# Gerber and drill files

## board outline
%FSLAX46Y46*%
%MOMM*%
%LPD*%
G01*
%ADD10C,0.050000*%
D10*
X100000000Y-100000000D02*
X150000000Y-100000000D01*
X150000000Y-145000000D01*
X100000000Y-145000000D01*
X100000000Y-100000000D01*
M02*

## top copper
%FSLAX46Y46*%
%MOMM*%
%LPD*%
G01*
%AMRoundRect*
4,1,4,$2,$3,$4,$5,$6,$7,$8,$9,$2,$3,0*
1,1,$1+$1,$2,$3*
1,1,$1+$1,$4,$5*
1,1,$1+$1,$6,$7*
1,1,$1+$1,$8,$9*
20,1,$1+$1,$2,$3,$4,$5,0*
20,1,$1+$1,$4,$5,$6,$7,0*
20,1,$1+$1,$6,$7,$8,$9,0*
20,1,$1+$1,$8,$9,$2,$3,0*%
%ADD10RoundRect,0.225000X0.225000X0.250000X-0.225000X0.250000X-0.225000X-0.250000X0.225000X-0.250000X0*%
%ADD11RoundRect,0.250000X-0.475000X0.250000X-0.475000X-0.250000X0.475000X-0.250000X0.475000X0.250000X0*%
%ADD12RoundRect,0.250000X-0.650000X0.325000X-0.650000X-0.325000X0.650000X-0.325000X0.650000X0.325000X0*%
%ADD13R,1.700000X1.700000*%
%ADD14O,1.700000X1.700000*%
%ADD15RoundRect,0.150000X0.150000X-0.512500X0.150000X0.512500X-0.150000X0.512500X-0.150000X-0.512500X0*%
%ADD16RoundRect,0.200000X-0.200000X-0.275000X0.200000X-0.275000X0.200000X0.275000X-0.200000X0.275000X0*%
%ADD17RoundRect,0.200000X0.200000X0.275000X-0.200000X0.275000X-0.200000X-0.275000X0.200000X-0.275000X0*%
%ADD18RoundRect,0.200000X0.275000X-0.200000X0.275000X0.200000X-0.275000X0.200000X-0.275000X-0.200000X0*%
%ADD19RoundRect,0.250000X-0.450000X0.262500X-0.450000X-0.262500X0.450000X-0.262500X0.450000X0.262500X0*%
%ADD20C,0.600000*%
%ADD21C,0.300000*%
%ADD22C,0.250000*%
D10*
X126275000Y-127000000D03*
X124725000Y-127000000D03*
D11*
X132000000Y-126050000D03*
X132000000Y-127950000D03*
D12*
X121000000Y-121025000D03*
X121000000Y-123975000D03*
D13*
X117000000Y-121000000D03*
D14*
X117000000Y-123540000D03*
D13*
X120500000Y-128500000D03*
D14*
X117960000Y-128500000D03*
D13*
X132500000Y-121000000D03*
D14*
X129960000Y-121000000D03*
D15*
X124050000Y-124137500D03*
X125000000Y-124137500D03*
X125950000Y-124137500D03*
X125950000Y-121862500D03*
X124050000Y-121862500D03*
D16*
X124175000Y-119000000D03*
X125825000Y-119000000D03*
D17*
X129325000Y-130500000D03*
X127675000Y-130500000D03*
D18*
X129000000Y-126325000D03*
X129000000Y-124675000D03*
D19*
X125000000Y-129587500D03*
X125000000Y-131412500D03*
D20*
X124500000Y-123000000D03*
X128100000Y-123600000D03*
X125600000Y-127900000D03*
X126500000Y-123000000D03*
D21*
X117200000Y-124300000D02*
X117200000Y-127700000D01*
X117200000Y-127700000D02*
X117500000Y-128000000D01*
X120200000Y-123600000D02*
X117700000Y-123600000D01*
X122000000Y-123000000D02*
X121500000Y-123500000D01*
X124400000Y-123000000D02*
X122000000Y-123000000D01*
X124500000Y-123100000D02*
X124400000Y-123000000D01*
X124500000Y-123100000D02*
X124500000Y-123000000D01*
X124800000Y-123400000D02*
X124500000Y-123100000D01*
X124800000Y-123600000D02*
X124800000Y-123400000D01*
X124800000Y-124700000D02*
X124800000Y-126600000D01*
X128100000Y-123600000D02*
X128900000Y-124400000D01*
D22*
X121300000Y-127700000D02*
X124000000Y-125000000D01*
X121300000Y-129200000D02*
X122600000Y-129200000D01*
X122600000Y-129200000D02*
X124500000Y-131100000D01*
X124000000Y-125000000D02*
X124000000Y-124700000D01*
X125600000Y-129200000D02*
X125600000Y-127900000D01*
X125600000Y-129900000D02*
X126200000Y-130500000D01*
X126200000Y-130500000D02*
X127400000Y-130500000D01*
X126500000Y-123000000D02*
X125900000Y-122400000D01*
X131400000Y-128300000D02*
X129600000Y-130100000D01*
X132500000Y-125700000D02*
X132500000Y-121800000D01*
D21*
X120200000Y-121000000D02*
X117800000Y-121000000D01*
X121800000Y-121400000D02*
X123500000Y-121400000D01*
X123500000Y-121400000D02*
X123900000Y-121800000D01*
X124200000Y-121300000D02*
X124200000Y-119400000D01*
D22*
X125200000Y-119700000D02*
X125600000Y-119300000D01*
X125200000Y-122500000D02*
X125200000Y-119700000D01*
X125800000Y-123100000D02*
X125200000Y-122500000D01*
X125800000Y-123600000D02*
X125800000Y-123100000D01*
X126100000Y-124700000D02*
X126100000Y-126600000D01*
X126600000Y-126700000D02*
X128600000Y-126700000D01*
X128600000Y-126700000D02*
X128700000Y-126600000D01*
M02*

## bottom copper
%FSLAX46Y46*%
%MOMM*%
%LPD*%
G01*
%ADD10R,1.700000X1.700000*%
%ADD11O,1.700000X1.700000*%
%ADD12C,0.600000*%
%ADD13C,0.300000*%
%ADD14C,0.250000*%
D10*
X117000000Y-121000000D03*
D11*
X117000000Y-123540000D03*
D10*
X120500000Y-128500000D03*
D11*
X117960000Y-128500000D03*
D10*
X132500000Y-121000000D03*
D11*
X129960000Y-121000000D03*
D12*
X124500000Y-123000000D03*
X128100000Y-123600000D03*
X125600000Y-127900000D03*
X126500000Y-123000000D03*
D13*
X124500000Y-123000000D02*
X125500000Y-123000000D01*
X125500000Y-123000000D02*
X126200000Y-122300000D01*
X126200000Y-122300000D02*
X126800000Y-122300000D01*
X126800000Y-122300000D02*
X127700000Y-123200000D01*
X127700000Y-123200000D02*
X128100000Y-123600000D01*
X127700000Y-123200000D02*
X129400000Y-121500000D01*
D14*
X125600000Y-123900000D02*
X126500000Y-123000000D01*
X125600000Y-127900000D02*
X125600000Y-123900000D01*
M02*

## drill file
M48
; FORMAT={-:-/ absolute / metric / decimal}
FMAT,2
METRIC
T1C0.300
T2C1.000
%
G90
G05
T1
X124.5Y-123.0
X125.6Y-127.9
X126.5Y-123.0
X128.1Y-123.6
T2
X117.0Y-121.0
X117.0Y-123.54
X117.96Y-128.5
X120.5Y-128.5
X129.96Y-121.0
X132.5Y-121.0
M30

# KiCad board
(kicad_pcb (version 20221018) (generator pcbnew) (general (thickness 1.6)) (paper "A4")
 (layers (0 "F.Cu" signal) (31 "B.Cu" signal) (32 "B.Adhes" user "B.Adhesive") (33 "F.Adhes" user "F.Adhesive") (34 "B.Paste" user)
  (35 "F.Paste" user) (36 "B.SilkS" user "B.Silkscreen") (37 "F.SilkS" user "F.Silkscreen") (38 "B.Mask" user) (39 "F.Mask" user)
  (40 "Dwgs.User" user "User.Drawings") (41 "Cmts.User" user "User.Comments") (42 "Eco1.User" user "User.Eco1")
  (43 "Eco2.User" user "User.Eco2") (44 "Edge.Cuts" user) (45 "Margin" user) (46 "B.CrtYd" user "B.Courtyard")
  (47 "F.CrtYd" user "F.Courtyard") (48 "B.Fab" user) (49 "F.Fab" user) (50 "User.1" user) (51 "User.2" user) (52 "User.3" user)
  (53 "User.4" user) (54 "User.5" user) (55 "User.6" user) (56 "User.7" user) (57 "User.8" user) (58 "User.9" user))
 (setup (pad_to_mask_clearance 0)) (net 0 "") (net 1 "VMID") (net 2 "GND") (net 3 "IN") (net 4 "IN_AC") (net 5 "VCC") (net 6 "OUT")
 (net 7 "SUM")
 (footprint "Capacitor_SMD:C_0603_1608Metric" (layer "F.Cu") (at 125.5 127 180)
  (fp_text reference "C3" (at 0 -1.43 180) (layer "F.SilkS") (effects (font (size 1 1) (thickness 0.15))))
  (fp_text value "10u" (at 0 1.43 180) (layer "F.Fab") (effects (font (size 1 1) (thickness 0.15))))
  (pad "1" smd roundrect (at -0.775 0 180) (size 0.9 0.95) (layers "F.Cu" "F.Paste" "F.Mask") (roundrect_rratio 0.25) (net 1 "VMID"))
  (pad "2" smd roundrect (at 0.775 0 180) (size 0.9 0.95) (layers "F.Cu" "F.Paste" "F.Mask") (roundrect_rratio 0.25) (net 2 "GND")))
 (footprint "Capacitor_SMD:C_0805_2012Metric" (layer "F.Cu") (at 132 127 -90)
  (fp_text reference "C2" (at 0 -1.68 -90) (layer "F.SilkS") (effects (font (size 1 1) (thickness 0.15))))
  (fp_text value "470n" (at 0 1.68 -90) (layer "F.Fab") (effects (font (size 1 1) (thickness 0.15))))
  (pad "1" smd roundrect (at -0.95 0 270) (size 1 1.45) (layers "F.Cu" "F.Paste" "F.Mask") (roundrect_rratio 0.25) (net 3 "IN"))
  (pad "2" smd roundrect (at 0.95 0 270) (size 1 1.45) (layers "F.Cu" "F.Paste" "F.Mask") (roundrect_rratio 0.25) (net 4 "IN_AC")))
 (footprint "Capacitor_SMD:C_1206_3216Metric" (layer "F.Cu") (at 121 122.5 -90)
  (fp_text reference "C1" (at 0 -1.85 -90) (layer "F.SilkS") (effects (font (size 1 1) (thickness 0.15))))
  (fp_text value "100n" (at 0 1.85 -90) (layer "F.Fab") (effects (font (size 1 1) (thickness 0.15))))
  (pad "1" smd roundrect (at -1.475 0 270) (size 1.15 1.8) (layers "F.Cu" "F.Paste" "F.Mask") (roundrect_rratio 0.217391) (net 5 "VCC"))
  (pad "2" smd roundrect (at 1.475 0 270) (size 1.15 1.8) (layers "F.Cu" "F.Paste" "F.Mask") (roundrect_rratio 0.217391) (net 2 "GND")))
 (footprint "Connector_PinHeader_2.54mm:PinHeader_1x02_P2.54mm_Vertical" (layer "F.Cu") (at 117 121)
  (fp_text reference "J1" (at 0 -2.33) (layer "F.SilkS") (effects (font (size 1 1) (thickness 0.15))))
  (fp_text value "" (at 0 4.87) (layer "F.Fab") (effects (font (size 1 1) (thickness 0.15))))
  (pad "1" thru_hole rect (at 0 0) (size 1.7 1.7) (drill 1) (layers "*.Cu" "*.Mask") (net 5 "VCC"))
  (pad "2" thru_hole oval (at 0 2.54) (size 1.7 1.7) (drill 1) (layers "*.Cu" "*.Mask") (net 2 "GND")))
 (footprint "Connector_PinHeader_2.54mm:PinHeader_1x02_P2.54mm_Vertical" (layer "F.Cu") (at 120.5 128.5 -90)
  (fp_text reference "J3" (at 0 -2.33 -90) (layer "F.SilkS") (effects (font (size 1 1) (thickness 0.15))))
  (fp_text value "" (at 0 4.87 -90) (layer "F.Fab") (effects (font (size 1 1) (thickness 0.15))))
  (pad "1" thru_hole rect (at 0 0 270) (size 1.7 1.7) (drill 1) (layers "*.Cu" "*.Mask") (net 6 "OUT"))
  (pad "2" thru_hole oval (at 0 2.54 270) (size 1.7 1.7) (drill 1) (layers "*.Cu" "*.Mask") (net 2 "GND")))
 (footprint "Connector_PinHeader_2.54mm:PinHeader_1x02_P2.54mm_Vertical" (layer "F.Cu") (at 132.5 121 -90)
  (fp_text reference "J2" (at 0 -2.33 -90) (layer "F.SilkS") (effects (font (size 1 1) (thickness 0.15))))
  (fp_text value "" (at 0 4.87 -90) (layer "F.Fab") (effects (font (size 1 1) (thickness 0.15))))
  (pad "1" thru_hole rect (at 0 0 270) (size 1.7 1.7) (drill 1) (layers "*.Cu" "*.Mask") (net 3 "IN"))
  (pad "2" thru_hole oval (at 0 2.54 270) (size 1.7 1.7) (drill 1) (layers "*.Cu" "*.Mask") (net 2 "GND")))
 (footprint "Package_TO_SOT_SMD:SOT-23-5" (layer "F.Cu") (at 125 123 90)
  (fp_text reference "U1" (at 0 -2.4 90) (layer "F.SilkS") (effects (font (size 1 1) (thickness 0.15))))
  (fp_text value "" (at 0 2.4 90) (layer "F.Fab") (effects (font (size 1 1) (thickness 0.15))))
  (pad "1" smd roundrect (at -1.1375 -0.95 90) (size 1.325 0.6) (layers "F.Cu" "F.Paste" "F.Mask") (roundrect_rratio 0.25) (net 6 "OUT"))
  (pad "2" smd roundrect (at -1.1375 0 90) (size 1.325 0.6) (layers "F.Cu" "F.Paste" "F.Mask") (roundrect_rratio 0.25) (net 2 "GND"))
  (pad "3" smd roundrect (at -1.1375 0.95 90) (size 1.325 0.6) (layers "F.Cu" "F.Paste" "F.Mask") (roundrect_rratio 0.25) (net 1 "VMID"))
  (pad "4" smd roundrect (at 1.1375 0.95 90) (size 1.325 0.6) (layers "F.Cu" "F.Paste" "F.Mask") (roundrect_rratio 0.25) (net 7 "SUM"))
  (pad "5" smd roundrect (at 1.1375 -0.95 90) (size 1.325 0.6) (layers "F.Cu" "F.Paste" "F.Mask") (roundrect_rratio 0.25) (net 5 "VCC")))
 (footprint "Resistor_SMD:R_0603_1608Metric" (layer "F.Cu") (at 125 119)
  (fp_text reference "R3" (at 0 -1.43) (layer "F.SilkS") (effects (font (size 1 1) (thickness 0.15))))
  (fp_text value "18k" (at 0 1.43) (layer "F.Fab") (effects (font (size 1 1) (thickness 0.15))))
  (pad "1" smd roundrect (at -0.825 0) (size 0.8 0.95) (layers "F.Cu" "F.Paste" "F.Mask") (roundrect_rratio 0.25) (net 5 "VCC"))
  (pad "2" smd roundrect (at 0.825 0) (size 0.8 0.95) (layers "F.Cu" "F.Paste" "F.Mask") (roundrect_rratio 0.25) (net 1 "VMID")))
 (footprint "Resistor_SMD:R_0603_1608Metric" (layer "F.Cu") (at 128.5 130.5 180)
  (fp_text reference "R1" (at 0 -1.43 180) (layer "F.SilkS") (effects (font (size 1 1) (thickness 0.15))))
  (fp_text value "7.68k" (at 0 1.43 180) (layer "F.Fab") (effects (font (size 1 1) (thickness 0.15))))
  (pad "1" smd roundrect (at -0.825 0 180) (size 0.8 0.95) (layers "F.Cu" "F.Paste" "F.Mask") (roundrect_rratio 0.25) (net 4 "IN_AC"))
  (pad "2" smd roundrect (at 0.825 0 180) (size 0.8 0.95) (layers "F.Cu" "F.Paste" "F.Mask") (roundrect_rratio 0.25) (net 7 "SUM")))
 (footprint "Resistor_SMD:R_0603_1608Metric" (layer "F.Cu") (at 129 125.5 90)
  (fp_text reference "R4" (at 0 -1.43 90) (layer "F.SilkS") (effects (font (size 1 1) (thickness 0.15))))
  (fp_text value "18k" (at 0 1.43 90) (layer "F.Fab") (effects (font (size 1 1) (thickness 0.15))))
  (pad "1" smd roundrect (at -0.825 0 90) (size 0.8 0.95) (layers "F.Cu" "F.Paste" "F.Mask") (roundrect_rratio 0.25) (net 1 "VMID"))
  (pad "2" smd roundrect (at 0.825 0 90) (size 0.8 0.95) (layers "F.Cu" "F.Paste" "F.Mask") (roundrect_rratio 0.25) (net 2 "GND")))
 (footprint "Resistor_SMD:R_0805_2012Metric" (layer "F.Cu") (at 125 130.5 -90)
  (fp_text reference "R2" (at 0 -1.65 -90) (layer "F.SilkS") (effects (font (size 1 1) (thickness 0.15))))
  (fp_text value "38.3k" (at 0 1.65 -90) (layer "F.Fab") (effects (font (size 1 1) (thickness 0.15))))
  (pad "1" smd roundrect (at -0.9125 0 270) (size 1.025 1.4) (layers "F.Cu" "F.Paste" "F.Mask") (roundrect_rratio 0.243902) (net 7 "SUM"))
  (pad "2" smd roundrect (at 0.9125 0 270) (size 1.025 1.4) (layers "F.Cu" "F.Paste" "F.Mask") (roundrect_rratio 0.243902) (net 6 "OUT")))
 (gr_rect (start 100 100) (end 150 145) (stroke (width 0.05) (type default)) (fill none) (layer "Edge.Cuts"))
 (segment (start 117.2 124.3) (end 117.2 127.7) (width 0.3) (layer "F.Cu") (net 2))
 (segment (start 117.2 127.7) (end 117.5 128) (width 0.3) (layer "F.Cu") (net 2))
 (segment (start 120.2 123.6) (end 117.7 123.6) (width 0.3) (layer "F.Cu") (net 2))
 (segment (start 122 123) (end 121.5 123.5) (width 0.3) (layer "F.Cu") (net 2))
 (segment (start 124.4 123) (end 122 123) (width 0.3) (layer "F.Cu") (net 2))
 (segment (start 124.5 123.1) (end 124.4 123) (width 0.3) (layer "F.Cu") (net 2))
 (segment (start 124.5 123.1) (end 124.5 123) (width 0.3) (layer "F.Cu") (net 2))
 (segment (start 124.8 123.4) (end 124.5 123.1) (width 0.3) (layer "F.Cu") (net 2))
 (segment (start 124.8 123.6) (end 124.8 123.4) (width 0.3) (layer "F.Cu") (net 2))
 (segment (start 124.8 124.7) (end 124.8 126.6) (width 0.3) (layer "F.Cu") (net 2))
 (segment (start 128.1 123.6) (end 128.9 124.4) (width 0.3) (layer "F.Cu") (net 2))
 (via (at 124.5 123) (size 0.6) (drill 0.3) (layers "F.Cu" "B.Cu") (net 2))
 (via (at 128.1 123.6) (size 0.6) (drill 0.3) (layers "F.Cu" "B.Cu") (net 2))
 (segment (start 121.3 127.7) (end 124 125) (width 0.25) (layer "F.Cu") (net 6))
 (segment (start 121.3 129.2) (end 122.6 129.2) (width 0.25) (layer "F.Cu") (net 6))
 (segment (start 122.6 129.2) (end 124.5 131.1) (width 0.25) (layer "F.Cu") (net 6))
 (segment (start 124 125) (end 124 124.7) (width 0.25) (layer "F.Cu") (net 6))
 (segment (start 124.5 123) (end 125.5 123) (width 0.3) (layer "B.Cu") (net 2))
 (segment (start 125.5 123) (end 126.2 122.3) (width 0.3) (layer "B.Cu") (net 2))
 (segment (start 125.6 129.2) (end 125.6 127.9) (width 0.25) (layer "F.Cu") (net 7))
 (segment (start 125.6 129.9) (end 126.2 130.5) (width 0.25) (layer "F.Cu") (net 7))
 (segment (start 126.2 122.3) (end 126.8 122.3) (width 0.3) (layer "B.Cu") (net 2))
 (segment (start 126.2 130.5) (end 127.4 130.5) (width 0.25) (layer "F.Cu") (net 7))
 (segment (start 126.5 123) (end 125.9 122.4) (width 0.25) (layer "F.Cu") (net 7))
 (segment (start 126.8 122.3) (end 127.7 123.2) (width 0.3) (layer "B.Cu") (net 2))
 (segment (start 127.7 123.2) (end 128.1 123.6) (width 0.3) (layer "B.Cu") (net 2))
 (segment (start 127.7 123.2) (end 129.4 121.5) (width 0.3) (layer "B.Cu") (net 2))
 (segment (start 131.4 128.3) (end 129.6 130.1) (width 0.25) (layer "F.Cu") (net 4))
 (segment (start 132.5 125.7) (end 132.5 121.8) (width 0.25) (layer "F.Cu") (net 3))
 (via (at 125.6 127.9) (size 0.6) (drill 0.3) (layers "F.Cu" "B.Cu") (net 7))
 (via (at 126.5 123) (size 0.6) (drill 0.3) (layers "F.Cu" "B.Cu") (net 7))
 (segment (start 120.2 121) (end 117.8 121) (width 0.3) (layer "F.Cu") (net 5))
 (segment (start 121.8 121.4) (end 123.5 121.4) (width 0.3) (layer "F.Cu") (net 5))
 (segment (start 123.5 121.4) (end 123.9 121.8) (width 0.3) (layer "F.Cu") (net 5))
 (segment (start 124.2 121.3) (end 124.2 119.4) (width 0.3) (layer "F.Cu") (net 5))
 (segment (start 125.2 119.7) (end 125.6 119.3) (width 0.25) (layer "F.Cu") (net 1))
 (segment (start 125.2 122.5) (end 125.2 119.7) (width 0.25) (layer "F.Cu") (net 1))
 (segment (start 125.6 123.9) (end 126.5 123) (width 0.25) (layer "B.Cu") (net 7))
 (segment (start 125.6 127.9) (end 125.6 123.9) (width 0.25) (layer "B.Cu") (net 7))
 (segment (start 125.8 123.1) (end 125.2 122.5) (width 0.25) (layer "F.Cu") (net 1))
 (segment (start 125.8 123.6) (end 125.8 123.1) (width 0.25) (layer "F.Cu") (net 1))
 (segment (start 126.1 124.7) (end 126.1 126.6) (width 0.25) (layer "F.Cu") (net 1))
 (segment (start 126.6 126.7) (end 128.6 126.7) (width 0.25) (layer "F.Cu") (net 1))
 (segment (start 128.6 126.7) (end 128.7 126.6) (width 0.25) (layer "F.Cu") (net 1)))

